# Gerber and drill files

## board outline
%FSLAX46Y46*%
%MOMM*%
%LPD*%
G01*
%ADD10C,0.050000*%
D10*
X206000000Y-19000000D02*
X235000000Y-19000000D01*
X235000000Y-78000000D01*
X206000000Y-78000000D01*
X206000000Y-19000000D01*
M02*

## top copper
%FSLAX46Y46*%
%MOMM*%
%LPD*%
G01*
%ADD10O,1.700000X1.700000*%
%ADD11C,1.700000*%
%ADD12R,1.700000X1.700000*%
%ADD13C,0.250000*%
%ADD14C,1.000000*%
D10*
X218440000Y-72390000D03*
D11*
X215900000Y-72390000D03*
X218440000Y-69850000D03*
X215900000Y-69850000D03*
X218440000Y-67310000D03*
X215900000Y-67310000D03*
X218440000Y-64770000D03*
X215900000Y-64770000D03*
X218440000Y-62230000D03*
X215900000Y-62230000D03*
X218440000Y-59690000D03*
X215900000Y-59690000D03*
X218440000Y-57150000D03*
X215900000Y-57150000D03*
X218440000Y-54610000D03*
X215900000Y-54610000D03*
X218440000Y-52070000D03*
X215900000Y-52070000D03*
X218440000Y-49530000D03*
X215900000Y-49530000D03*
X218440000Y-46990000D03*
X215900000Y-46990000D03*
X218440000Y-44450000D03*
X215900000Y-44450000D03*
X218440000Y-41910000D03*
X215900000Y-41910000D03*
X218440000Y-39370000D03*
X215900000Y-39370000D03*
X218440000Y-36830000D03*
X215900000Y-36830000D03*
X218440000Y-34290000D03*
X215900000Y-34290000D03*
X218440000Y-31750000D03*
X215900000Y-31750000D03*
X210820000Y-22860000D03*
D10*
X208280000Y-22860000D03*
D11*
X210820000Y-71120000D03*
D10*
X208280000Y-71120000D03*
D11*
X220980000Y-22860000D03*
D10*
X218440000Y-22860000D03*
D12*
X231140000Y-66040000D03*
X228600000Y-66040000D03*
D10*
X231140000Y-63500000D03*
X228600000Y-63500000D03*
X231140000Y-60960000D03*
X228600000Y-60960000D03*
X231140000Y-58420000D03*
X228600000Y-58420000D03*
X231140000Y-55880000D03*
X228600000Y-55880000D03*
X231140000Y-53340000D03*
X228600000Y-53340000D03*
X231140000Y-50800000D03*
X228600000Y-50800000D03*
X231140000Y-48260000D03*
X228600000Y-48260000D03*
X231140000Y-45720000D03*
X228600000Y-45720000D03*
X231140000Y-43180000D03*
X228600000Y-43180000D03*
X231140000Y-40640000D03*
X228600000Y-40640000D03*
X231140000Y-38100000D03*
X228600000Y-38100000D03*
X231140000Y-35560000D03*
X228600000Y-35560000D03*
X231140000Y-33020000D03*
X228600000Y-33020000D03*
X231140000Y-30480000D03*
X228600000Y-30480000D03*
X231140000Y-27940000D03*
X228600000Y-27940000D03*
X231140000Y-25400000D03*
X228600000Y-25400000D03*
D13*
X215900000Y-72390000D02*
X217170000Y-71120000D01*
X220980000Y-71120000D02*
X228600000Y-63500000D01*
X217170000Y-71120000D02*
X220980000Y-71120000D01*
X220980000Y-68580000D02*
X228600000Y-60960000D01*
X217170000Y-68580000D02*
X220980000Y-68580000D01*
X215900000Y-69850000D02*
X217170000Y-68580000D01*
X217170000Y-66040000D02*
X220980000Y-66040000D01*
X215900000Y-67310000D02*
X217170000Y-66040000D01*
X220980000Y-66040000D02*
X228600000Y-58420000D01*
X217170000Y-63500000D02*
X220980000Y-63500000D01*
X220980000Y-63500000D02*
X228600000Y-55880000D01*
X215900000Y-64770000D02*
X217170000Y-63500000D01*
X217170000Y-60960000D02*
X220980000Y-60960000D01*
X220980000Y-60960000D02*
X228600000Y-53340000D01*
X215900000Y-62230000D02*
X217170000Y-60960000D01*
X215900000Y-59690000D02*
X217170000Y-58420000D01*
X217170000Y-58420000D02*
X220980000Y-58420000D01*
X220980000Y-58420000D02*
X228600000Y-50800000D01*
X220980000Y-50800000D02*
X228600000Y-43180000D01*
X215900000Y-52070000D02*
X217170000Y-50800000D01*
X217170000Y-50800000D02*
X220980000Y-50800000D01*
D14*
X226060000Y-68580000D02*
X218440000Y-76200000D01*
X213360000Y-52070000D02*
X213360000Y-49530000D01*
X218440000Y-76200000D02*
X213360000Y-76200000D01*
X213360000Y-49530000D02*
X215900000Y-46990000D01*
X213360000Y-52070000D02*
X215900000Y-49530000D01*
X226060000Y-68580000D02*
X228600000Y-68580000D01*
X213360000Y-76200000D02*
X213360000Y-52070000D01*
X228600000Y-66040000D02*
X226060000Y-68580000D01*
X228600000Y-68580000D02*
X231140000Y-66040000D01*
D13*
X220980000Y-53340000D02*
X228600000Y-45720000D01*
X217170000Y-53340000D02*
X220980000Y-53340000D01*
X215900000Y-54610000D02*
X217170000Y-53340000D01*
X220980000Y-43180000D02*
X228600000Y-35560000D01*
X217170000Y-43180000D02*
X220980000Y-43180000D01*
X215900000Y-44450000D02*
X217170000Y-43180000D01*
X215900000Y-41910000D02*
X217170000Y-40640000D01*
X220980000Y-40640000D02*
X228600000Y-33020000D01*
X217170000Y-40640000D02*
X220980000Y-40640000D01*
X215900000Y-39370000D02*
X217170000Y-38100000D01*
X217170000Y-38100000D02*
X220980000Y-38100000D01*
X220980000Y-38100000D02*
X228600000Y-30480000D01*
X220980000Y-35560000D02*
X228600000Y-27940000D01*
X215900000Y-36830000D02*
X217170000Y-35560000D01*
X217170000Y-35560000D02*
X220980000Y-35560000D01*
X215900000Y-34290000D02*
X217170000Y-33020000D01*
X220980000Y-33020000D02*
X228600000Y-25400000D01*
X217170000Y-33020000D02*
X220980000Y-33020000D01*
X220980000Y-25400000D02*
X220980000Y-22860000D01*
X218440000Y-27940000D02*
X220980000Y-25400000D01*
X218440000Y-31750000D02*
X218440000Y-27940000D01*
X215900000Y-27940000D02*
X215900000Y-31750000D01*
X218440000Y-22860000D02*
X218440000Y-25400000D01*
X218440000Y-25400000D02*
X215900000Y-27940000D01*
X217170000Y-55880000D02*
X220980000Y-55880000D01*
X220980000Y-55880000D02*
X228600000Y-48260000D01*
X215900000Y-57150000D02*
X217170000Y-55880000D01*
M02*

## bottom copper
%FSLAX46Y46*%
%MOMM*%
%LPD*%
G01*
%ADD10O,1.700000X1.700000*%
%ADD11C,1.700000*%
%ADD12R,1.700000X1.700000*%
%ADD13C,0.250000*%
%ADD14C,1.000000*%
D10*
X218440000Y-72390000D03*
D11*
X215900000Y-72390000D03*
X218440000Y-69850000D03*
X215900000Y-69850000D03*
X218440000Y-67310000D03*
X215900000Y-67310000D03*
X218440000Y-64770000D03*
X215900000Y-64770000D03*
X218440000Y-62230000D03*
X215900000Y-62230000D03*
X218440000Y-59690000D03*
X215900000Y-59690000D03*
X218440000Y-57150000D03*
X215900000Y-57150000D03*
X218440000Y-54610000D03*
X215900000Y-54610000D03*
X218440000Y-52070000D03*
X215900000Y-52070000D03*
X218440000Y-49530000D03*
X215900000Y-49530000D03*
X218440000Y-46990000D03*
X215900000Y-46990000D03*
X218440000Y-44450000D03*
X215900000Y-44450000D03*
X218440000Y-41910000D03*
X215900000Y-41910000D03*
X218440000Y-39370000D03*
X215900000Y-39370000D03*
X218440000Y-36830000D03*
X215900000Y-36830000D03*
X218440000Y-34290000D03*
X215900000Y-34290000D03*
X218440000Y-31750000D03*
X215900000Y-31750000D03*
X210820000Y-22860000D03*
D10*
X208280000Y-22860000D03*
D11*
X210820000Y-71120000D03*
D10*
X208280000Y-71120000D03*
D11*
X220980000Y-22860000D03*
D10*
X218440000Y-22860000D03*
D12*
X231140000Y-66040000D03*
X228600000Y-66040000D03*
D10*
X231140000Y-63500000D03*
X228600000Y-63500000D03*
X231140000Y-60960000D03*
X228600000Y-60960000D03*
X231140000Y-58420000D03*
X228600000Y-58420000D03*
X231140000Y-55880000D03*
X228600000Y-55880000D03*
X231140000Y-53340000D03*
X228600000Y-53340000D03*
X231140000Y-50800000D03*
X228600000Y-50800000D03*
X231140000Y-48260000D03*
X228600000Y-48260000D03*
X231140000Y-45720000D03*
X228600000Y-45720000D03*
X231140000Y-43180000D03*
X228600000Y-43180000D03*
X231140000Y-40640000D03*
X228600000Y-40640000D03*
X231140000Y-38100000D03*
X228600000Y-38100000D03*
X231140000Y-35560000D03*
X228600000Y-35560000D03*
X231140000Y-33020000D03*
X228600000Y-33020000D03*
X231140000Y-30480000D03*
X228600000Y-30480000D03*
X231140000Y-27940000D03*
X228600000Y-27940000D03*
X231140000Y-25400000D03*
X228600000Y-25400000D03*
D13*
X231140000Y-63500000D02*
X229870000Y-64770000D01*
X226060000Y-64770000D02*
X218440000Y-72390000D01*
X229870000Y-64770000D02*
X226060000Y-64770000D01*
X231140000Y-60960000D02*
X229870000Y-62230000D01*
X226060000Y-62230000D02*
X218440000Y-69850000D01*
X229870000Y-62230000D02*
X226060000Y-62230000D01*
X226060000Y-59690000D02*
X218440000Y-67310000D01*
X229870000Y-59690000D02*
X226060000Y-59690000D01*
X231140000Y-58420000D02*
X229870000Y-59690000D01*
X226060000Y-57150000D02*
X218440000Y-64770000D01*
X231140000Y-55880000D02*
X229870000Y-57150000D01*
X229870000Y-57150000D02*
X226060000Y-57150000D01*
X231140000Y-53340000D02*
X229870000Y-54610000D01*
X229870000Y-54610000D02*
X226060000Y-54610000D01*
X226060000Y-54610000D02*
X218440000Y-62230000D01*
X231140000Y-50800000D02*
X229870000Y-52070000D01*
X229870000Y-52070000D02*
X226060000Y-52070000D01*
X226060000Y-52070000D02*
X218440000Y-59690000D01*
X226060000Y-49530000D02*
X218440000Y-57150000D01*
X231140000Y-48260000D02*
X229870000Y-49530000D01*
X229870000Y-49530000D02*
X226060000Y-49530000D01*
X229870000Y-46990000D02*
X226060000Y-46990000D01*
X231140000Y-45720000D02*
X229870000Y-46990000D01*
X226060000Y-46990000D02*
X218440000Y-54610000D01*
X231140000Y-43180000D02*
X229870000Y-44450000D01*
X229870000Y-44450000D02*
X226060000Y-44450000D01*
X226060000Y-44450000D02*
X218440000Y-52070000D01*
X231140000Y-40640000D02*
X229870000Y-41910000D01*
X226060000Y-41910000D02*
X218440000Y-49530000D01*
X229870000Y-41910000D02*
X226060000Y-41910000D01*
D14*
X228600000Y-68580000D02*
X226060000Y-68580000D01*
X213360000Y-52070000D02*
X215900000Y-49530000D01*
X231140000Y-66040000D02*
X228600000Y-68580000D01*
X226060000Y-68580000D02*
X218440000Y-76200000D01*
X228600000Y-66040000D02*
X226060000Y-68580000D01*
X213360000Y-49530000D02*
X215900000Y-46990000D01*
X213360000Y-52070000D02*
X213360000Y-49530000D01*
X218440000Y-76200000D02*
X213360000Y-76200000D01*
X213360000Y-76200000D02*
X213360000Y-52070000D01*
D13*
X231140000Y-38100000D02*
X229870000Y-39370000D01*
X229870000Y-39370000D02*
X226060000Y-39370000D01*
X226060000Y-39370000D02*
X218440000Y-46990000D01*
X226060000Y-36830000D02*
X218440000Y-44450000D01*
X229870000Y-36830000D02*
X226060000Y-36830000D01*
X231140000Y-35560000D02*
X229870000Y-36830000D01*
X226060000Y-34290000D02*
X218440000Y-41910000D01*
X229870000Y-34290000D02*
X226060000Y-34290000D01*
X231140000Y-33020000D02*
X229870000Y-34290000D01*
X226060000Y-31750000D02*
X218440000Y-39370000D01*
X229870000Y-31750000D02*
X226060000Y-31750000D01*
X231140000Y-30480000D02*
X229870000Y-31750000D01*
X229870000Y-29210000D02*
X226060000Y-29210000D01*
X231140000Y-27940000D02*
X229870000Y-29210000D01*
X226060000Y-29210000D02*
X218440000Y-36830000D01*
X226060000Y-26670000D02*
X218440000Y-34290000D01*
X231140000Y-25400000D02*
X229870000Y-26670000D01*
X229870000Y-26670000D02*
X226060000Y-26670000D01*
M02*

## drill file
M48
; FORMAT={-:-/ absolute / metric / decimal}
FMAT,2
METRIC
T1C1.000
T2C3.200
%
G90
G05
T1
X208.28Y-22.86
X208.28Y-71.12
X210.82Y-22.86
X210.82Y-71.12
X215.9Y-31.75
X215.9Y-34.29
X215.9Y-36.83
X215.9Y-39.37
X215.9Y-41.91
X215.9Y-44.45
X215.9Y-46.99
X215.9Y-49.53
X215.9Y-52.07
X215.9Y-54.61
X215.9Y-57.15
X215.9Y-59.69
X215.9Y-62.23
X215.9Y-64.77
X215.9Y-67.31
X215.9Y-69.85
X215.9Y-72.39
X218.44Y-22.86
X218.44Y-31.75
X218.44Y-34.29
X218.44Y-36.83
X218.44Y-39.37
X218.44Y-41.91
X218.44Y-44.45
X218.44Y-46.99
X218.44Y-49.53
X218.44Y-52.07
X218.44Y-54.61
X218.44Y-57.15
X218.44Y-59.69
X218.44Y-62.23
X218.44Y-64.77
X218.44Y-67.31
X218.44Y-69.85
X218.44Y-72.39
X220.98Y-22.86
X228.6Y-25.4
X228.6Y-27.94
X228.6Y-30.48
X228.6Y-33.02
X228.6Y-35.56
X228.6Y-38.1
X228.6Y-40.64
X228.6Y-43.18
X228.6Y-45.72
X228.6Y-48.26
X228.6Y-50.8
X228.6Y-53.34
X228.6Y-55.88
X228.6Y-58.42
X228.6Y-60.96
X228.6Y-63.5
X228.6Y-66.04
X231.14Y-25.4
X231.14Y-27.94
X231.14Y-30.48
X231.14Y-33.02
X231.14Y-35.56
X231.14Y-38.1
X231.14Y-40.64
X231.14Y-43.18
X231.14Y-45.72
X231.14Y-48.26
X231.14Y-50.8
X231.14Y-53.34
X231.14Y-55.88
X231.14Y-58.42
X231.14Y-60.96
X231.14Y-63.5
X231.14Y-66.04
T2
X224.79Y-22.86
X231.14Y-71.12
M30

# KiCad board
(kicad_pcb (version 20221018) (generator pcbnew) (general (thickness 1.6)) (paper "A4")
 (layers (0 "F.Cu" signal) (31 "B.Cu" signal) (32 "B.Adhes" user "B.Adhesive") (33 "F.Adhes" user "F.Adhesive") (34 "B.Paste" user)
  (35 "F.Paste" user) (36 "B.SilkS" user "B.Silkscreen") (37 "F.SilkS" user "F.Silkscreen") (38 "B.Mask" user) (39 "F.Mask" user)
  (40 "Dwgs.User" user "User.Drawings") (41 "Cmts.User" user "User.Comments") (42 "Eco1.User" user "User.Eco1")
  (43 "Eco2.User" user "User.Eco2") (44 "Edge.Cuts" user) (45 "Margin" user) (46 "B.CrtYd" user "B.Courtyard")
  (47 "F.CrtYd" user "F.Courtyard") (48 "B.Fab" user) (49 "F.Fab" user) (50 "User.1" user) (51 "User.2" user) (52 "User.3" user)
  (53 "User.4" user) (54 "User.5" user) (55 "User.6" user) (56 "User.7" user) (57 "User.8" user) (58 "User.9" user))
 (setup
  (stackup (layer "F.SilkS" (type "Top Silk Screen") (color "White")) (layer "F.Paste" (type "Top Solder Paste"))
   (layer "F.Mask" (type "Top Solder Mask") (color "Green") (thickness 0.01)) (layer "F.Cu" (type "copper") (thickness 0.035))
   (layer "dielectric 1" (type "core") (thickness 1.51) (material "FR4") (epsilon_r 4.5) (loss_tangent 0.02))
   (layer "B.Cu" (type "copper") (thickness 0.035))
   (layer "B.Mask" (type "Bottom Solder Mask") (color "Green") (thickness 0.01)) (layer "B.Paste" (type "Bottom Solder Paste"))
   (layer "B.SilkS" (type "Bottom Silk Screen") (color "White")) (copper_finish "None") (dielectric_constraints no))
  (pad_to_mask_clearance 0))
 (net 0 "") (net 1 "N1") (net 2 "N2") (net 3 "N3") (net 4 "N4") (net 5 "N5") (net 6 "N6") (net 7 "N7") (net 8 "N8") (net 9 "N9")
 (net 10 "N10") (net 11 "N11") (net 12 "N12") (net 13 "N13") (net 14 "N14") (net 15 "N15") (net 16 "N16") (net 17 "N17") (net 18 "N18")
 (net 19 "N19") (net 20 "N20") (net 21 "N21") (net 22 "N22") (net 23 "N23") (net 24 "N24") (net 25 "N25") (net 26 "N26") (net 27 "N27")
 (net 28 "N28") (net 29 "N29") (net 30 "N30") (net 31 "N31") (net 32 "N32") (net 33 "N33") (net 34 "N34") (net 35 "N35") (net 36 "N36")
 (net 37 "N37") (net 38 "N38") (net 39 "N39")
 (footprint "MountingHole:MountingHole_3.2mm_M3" (layer "F.Cu") (at 224.79 22.86)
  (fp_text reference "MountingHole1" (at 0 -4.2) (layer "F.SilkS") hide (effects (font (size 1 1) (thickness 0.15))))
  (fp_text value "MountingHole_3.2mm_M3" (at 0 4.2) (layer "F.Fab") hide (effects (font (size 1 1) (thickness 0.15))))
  (pad "" np_thru_hole circle (at 0 0) (size 3.2 3.2) (drill 3.2) (layers "F&B.Cu" "*.Mask")))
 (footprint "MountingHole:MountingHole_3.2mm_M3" (layer "F.Cu") (at 231.14 71.12)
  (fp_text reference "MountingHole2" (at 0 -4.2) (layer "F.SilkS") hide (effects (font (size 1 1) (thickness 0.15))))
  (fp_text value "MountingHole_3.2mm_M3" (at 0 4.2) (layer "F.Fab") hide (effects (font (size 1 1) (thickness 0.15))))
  (pad "" np_thru_hole circle (at 0 0) (size 3.2 3.2) (drill 3.2) (layers "*.Cu" "*.Mask")))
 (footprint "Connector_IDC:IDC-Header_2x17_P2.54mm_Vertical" (layer "F.Cu") (at 218.44 72.39 180)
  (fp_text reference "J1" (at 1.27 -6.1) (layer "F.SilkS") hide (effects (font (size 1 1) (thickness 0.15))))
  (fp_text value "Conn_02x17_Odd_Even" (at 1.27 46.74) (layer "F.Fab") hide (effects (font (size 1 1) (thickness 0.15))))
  (pad "1" thru_hole oval (at 0 0 180) (size 1.7 1.7) (drill 1) (layers "*.Cu" "*.Mask") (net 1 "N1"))
  (pad "2" thru_hole circle (at 2.54 0 180) (size 1.7 1.7) (drill 1) (layers "*.Cu" "*.Mask") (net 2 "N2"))
  (pad "3" thru_hole circle (at 0 2.54 180) (size 1.7 1.7) (drill 1) (layers "*.Cu" "*.Mask") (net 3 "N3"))
  (pad "4" thru_hole circle (at 2.54 2.54 180) (size 1.7 1.7) (drill 1) (layers "*.Cu" "*.Mask") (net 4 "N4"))
  (pad "5" thru_hole circle (at 0 5.08 180) (size 1.7 1.7) (drill 1) (layers "*.Cu" "*.Mask") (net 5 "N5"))
  (pad "6" thru_hole circle (at 2.54 5.08 180) (size 1.7 1.7) (drill 1) (layers "*.Cu" "*.Mask") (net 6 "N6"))
  (pad "7" thru_hole circle (at 0 7.62 180) (size 1.7 1.7) (drill 1) (layers "*.Cu" "*.Mask") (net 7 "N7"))
  (pad "8" thru_hole circle (at 2.54 7.62 180) (size 1.7 1.7) (drill 1) (layers "*.Cu" "*.Mask") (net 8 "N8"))
  (pad "9" thru_hole circle (at 0 10.16 180) (size 1.7 1.7) (drill 1) (layers "*.Cu" "*.Mask") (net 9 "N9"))
  (pad "10" thru_hole circle (at 2.54 10.16 180) (size 1.7 1.7) (drill 1) (layers "*.Cu" "*.Mask") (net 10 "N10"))
  (pad "11" thru_hole circle (at 0 12.7 180) (size 1.7 1.7) (drill 1) (layers "*.Cu" "*.Mask") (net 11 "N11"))
  (pad "12" thru_hole circle (at 2.54 12.7 180) (size 1.7 1.7) (drill 1) (layers "*.Cu" "*.Mask") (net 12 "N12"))
  (pad "13" thru_hole circle (at 0 15.24 180) (size 1.7 1.7) (drill 1) (layers "*.Cu" "*.Mask") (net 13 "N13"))
  (pad "14" thru_hole circle (at 2.54 15.24 180) (size 1.7 1.7) (drill 1) (layers "*.Cu" "*.Mask") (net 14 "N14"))
  (pad "15" thru_hole circle (at 0 17.78 180) (size 1.7 1.7) (drill 1) (layers "*.Cu" "*.Mask") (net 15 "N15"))
  (pad "16" thru_hole circle (at 2.54 17.78 180) (size 1.7 1.7) (drill 1) (layers "*.Cu" "*.Mask") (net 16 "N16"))
  (pad "17" thru_hole circle (at 0 20.32 180) (size 1.7 1.7) (drill 1) (layers "*.Cu" "*.Mask") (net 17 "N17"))
  (pad "18" thru_hole circle (at 2.54 20.32 180) (size 1.7 1.7) (drill 1) (layers "*.Cu" "*.Mask") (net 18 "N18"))
  (pad "19" thru_hole circle (at 0 22.86 180) (size 1.7 1.7) (drill 1) (layers "*.Cu" "*.Mask") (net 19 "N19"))
  (pad "20" thru_hole circle (at 2.54 22.86 180) (size 1.7 1.7) (drill 1) (layers "*.Cu" "*.Mask") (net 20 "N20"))
  (pad "21" thru_hole circle (at 0 25.4 180) (size 1.7 1.7) (drill 1) (layers "*.Cu" "*.Mask") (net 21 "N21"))
  (pad "22" thru_hole circle (at 2.54 25.4 180) (size 1.7 1.7) (drill 1) (layers "*.Cu" "*.Mask") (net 20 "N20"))
  (pad "23" thru_hole circle (at 0 27.94 180) (size 1.7 1.7) (drill 1) (layers "*.Cu" "*.Mask") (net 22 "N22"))
  (pad "24" thru_hole circle (at 2.54 27.94 180) (size 1.7 1.7) (drill 1) (layers "*.Cu" "*.Mask") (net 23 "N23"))
  (pad "25" thru_hole circle (at 0 30.48 180) (size 1.7 1.7) (drill 1) (layers "*.Cu" "*.Mask") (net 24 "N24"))
  (pad "26" thru_hole circle (at 2.54 30.48 180) (size 1.7 1.7) (drill 1) (layers "*.Cu" "*.Mask") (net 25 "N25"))
  (pad "27" thru_hole circle (at 0 33.02 180) (size 1.7 1.7) (drill 1) (layers "*.Cu" "*.Mask") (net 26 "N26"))
  (pad "28" thru_hole circle (at 2.54 33.02 180) (size 1.7 1.7) (drill 1) (layers "*.Cu" "*.Mask") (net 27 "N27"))
  (pad "29" thru_hole circle (at 0 35.56 180) (size 1.7 1.7) (drill 1) (layers "*.Cu" "*.Mask") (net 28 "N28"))
  (pad "30" thru_hole circle (at 2.54 35.56 180) (size 1.7 1.7) (drill 1) (layers "*.Cu" "*.Mask") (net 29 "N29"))
  (pad "31" thru_hole circle (at 0 38.1 180) (size 1.7 1.7) (drill 1) (layers "*.Cu" "*.Mask") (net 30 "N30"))
  (pad "32" thru_hole circle (at 2.54 38.1 180) (size 1.7 1.7) (drill 1) (layers "*.Cu" "*.Mask") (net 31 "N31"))
  (pad "33" thru_hole circle (at 0 40.64 180) (size 1.7 1.7) (drill 1) (layers "*.Cu" "*.Mask") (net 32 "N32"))
  (pad "34" thru_hole circle (at 2.54 40.64 180) (size 1.7 1.7) (drill 1) (layers "*.Cu" "*.Mask") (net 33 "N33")))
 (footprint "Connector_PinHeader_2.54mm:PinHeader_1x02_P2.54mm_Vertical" (layer "B.Cu") (at 210.82 22.86 90)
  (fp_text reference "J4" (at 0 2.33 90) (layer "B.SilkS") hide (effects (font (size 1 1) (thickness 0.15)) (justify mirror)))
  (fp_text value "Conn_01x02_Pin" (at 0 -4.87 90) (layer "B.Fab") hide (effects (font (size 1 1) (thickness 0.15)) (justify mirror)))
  (pad "1" thru_hole circle (at 0 0 90) (size 1.7 1.7) (drill 1) (layers "*.Cu" "*.Mask") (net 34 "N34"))
  (pad "2" thru_hole oval (at 0 -2.54 90) (size 1.7 1.7) (drill 1) (layers "*.Cu" "*.Mask") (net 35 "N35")))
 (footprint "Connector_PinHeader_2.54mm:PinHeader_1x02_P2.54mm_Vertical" (layer "B.Cu") (at 210.82 71.12 90)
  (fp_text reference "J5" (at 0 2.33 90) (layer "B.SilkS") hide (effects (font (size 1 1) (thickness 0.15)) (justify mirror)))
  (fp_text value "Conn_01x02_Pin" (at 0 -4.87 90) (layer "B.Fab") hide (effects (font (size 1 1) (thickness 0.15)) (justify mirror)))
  (pad "1" thru_hole circle (at 0 0 90) (size 1.7 1.7) (drill 1) (layers "*.Cu" "*.Mask") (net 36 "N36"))
  (pad "2" thru_hole oval (at 0 -2.54 90) (size 1.7 1.7) (drill 1) (layers "*.Cu" "*.Mask") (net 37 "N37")))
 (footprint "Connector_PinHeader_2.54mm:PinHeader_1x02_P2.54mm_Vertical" (layer "B.Cu") (at 220.98 22.86 90)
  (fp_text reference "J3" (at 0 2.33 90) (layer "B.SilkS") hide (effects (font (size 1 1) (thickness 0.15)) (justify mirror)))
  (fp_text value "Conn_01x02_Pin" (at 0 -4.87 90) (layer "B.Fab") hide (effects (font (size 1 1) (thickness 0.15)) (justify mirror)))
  (pad "1" thru_hole circle (at 0 0 90) (size 1.7 1.7) (drill 1) (layers "*.Cu" "*.Mask") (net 32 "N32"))
  (pad "2" thru_hole oval (at 0 -2.54 90) (size 1.7 1.7) (drill 1) (layers "*.Cu" "*.Mask") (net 33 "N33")))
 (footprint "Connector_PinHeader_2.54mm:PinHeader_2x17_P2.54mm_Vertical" (layer "B.Cu") (at 228.6 66.04)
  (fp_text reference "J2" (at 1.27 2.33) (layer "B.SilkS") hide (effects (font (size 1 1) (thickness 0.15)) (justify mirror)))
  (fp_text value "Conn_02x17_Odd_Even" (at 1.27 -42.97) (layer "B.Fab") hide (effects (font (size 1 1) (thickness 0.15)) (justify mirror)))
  (pad "1" thru_hole rect (at 2.54 0) (size 1.7 1.7) (drill 1) (layers "*.Cu" "*.Mask") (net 20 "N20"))
  (pad "2" thru_hole rect (at 0 0) (size 1.7 1.7) (drill 1) (layers "*.Cu" "*.Mask") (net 20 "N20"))
  (pad "3" thru_hole oval (at 2.54 -2.54) (size 1.7 1.7) (drill 1) (layers "*.Cu" "*.Mask") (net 1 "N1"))
  (pad "4" thru_hole oval (at 0 -2.54) (size 1.7 1.7) (drill 1) (layers "*.Cu" "*.Mask") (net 2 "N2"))
  (pad "5" thru_hole oval (at 2.54 -5.08) (size 1.7 1.7) (drill 1) (layers "*.Cu" "*.Mask") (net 3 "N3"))
  (pad "6" thru_hole oval (at 0 -5.08) (size 1.7 1.7) (drill 1) (layers "*.Cu" "*.Mask") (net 4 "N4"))
  (pad "7" thru_hole oval (at 2.54 -7.62) (size 1.7 1.7) (drill 1) (layers "*.Cu" "*.Mask") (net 5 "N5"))
  (pad "8" thru_hole oval (at 0 -7.62) (size 1.7 1.7) (drill 1) (layers "*.Cu" "*.Mask") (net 6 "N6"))
  (pad "9" thru_hole oval (at 2.54 -10.16) (size 1.7 1.7) (drill 1) (layers "*.Cu" "*.Mask") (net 7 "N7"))
  (pad "10" thru_hole oval (at 0 -10.16) (size 1.7 1.7) (drill 1) (layers "*.Cu" "*.Mask") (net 8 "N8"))
  (pad "11" thru_hole oval (at 2.54 -12.7) (size 1.7 1.7) (drill 1) (layers "*.Cu" "*.Mask") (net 9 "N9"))
  (pad "12" thru_hole oval (at 0 -12.7) (size 1.7 1.7) (drill 1) (layers "*.Cu" "*.Mask") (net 10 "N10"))
  (pad "13" thru_hole oval (at 2.54 -15.24) (size 1.7 1.7) (drill 1) (layers "*.Cu" "*.Mask") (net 11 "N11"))
  (pad "14" thru_hole oval (at 0 -15.24) (size 1.7 1.7) (drill 1) (layers "*.Cu" "*.Mask") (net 12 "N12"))
  (pad "15" thru_hole oval (at 2.54 -17.78) (size 1.7 1.7) (drill 1) (layers "*.Cu" "*.Mask") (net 13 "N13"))
  (pad "16" thru_hole oval (at 0 -17.78) (size 1.7 1.7) (drill 1) (layers "*.Cu" "*.Mask") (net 14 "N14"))
  (pad "17" thru_hole oval (at 2.54 -20.32) (size 1.7 1.7) (drill 1) (layers "*.Cu" "*.Mask") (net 15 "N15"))
  (pad "18" thru_hole oval (at 0 -20.32) (size 1.7 1.7) (drill 1) (layers "*.Cu" "*.Mask") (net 16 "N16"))
  (pad "19" thru_hole oval (at 2.54 -22.86) (size 1.7 1.7) (drill 1) (layers "*.Cu" "*.Mask") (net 17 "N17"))
  (pad "20" thru_hole oval (at 0 -22.86) (size 1.7 1.7) (drill 1) (layers "*.Cu" "*.Mask") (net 18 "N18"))
  (pad "21" thru_hole oval (at 2.54 -25.4) (size 1.7 1.7) (drill 1) (layers "*.Cu" "*.Mask") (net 19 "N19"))
  (pad "22" thru_hole oval (at 0 -25.4) (size 1.7 1.7) (drill 1) (layers "*.Cu" "*.Mask") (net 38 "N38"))
  (pad "23" thru_hole oval (at 2.54 -27.94) (size 1.7 1.7) (drill 1) (layers "*.Cu" "*.Mask") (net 21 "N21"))
  (pad "24" thru_hole oval (at 0 -27.94) (size 1.7 1.7) (drill 1) (layers "*.Cu" "*.Mask") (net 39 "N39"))
  (pad "25" thru_hole oval (at 2.54 -30.48) (size 1.7 1.7) (drill 1) (layers "*.Cu" "*.Mask") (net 22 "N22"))
  (pad "26" thru_hole oval (at 0 -30.48) (size 1.7 1.7) (drill 1) (layers "*.Cu" "*.Mask") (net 23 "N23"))
  (pad "27" thru_hole oval (at 2.54 -33.02) (size 1.7 1.7) (drill 1) (layers "*.Cu" "*.Mask") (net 24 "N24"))
  (pad "28" thru_hole oval (at 0 -33.02) (size 1.7 1.7) (drill 1) (layers "*.Cu" "*.Mask") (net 25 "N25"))
  (pad "29" thru_hole oval (at 2.54 -35.56) (size 1.7 1.7) (drill 1) (layers "*.Cu" "*.Mask") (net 26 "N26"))
  (pad "30" thru_hole oval (at 0 -35.56) (size 1.7 1.7) (drill 1) (layers "*.Cu" "*.Mask") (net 27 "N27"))
  (pad "31" thru_hole oval (at 2.54 -38.1) (size 1.7 1.7) (drill 1) (layers "*.Cu" "*.Mask") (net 28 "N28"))
  (pad "32" thru_hole oval (at 0 -38.1) (size 1.7 1.7) (drill 1) (layers "*.Cu" "*.Mask") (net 29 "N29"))
  (pad "33" thru_hole oval (at 2.54 -40.64) (size 1.7 1.7) (drill 1) (layers "*.Cu" "*.Mask") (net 30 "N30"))
  (pad "34" thru_hole oval (at 0 -40.64) (size 1.7 1.7) (drill 1) (layers "*.Cu" "*.Mask") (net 31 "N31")))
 (gr_rect (start 206 19) (end 235 78) (stroke (width 0.05) (type default)) (fill none) (layer "Edge.Cuts"))
 (segment (start 231.14 63.5) (end 229.87 64.77) (width 0.25) (layer "B.Cu") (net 1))
 (segment (start 226.06 64.77) (end 218.44 72.39) (width 0.25) (layer "B.Cu") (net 1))
 (segment (start 229.87 64.77) (end 226.06 64.77) (width 0.25) (layer "B.Cu") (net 1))
 (segment (start 215.9 72.39) (end 217.17 71.12) (width 0.25) (layer "F.Cu") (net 2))
 (segment (start 220.98 71.12) (end 228.6 63.5) (width 0.25) (layer "F.Cu") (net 2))
 (segment (start 217.17 71.12) (end 220.98 71.12) (width 0.25) (layer "F.Cu") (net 2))
 (segment (start 231.14 60.96) (end 229.87 62.23) (width 0.25) (layer "B.Cu") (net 3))
 (segment (start 226.06 62.23) (end 218.44 69.85) (width 0.25) (layer "B.Cu") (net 3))
 (segment (start 229.87 62.23) (end 226.06 62.23) (width 0.25) (layer "B.Cu") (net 3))
 (segment (start 220.98 68.58) (end 228.6 60.96) (width 0.25) (layer "F.Cu") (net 4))
 (segment (start 217.17 68.58) (end 220.98 68.58) (width 0.25) (layer "F.Cu") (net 4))
 (segment (start 215.9 69.85) (end 217.17 68.58) (width 0.25) (layer "F.Cu") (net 4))
 (segment (start 226.06 59.69) (end 218.44 67.31) (width 0.25) (layer "B.Cu") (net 5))
 (segment (start 229.87 59.69) (end 226.06 59.69) (width 0.25) (layer "B.Cu") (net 5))
 (segment (start 231.14 58.42) (end 229.87 59.69) (width 0.25) (layer "B.Cu") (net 5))
 (segment (start 217.17 66.04) (end 220.98 66.04) (width 0.25) (layer "F.Cu") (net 6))
 (segment (start 215.9 67.31) (end 217.17 66.04) (width 0.25) (layer "F.Cu") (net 6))
 (segment (start 220.98 66.04) (end 228.6 58.42) (width 0.25) (layer "F.Cu") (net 6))
 (segment (start 226.06 57.15) (end 218.44 64.77) (width 0.25) (layer "B.Cu") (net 7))
 (segment (start 231.14 55.88) (end 229.87 57.15) (width 0.25) (layer "B.Cu") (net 7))
 (segment (start 229.87 57.15) (end 226.06 57.15) (width 0.25) (layer "B.Cu") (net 7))
 (segment (start 217.17 63.5) (end 220.98 63.5) (width 0.25) (layer "F.Cu") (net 8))
 (segment (start 220.98 63.5) (end 228.6 55.88) (width 0.25) (layer "F.Cu") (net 8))
 (segment (start 215.9 64.77) (end 217.17 63.5) (width 0.25) (layer "F.Cu") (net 8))
 (segment (start 231.14 53.34) (end 229.87 54.61) (width 0.25) (layer "B.Cu") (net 9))
 (segment (start 229.87 54.61) (end 226.06 54.61) (width 0.25) (layer "B.Cu") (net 9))
 (segment (start 226.06 54.61) (end 218.44 62.23) (width 0.25) (layer "B.Cu") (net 9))
 (segment (start 217.17 60.96) (end 220.98 60.96) (width 0.25) (layer "F.Cu") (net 10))
 (segment (start 220.98 60.96) (end 228.6 53.34) (width 0.25) (layer "F.Cu") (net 10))
 (segment (start 215.9 62.23) (end 217.17 60.96) (width 0.25) (layer "F.Cu") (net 10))
 (segment (start 231.14 50.8) (end 229.87 52.07) (width 0.25) (layer "B.Cu") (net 11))
 (segment (start 229.87 52.07) (end 226.06 52.07) (width 0.25) (layer "B.Cu") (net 11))
 (segment (start 226.06 52.07) (end 218.44 59.69) (width 0.25) (layer "B.Cu") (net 11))
 (segment (start 215.9 59.69) (end 217.17 58.42) (width 0.25) (layer "F.Cu") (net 12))
 (segment (start 217.17 58.42) (end 220.98 58.42) (width 0.25) (layer "F.Cu") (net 12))
 (segment (start 220.98 58.42) (end 228.6 50.8) (width 0.25) (layer "F.Cu") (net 12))
 (segment (start 226.06 49.53) (end 218.44 57.15) (width 0.25) (layer "B.Cu") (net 13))
 (segment (start 231.14 48.26) (end 229.87 49.53) (width 0.25) (layer "B.Cu") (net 13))
 (segment (start 229.87 49.53) (end 226.06 49.53) (width 0.25) (layer "B.Cu") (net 13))
 (segment (start 229.87 46.99) (end 226.06 46.99) (width 0.25) (layer "B.Cu") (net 15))
 (segment (start 231.14 45.72) (end 229.87 46.99) (width 0.25) (layer "B.Cu") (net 15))
 (segment (start 226.06 46.99) (end 218.44 54.61) (width 0.25) (layer "B.Cu") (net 15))
 (segment (start 231.14 43.18) (end 229.87 44.45) (width 0.25) (layer "B.Cu") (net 17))
 (segment (start 229.87 44.45) (end 226.06 44.45) (width 0.25) (layer "B.Cu") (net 17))
 (segment (start 226.06 44.45) (end 218.44 52.07) (width 0.25) (layer "B.Cu") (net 17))
 (segment (start 220.98 50.8) (end 228.6 43.18) (width 0.25) (layer "F.Cu") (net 18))
 (segment (start 215.9 52.07) (end 217.17 50.8) (width 0.25) (layer "F.Cu") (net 18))
 (segment (start 217.17 50.8) (end 220.98 50.8) (width 0.25) (layer "F.Cu") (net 18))
 (segment (start 231.14 40.64) (end 229.87 41.91) (width 0.25) (layer "B.Cu") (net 19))
 (segment (start 226.06 41.91) (end 218.44 49.53) (width 0.25) (layer "B.Cu") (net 19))
 (segment (start 229.87 41.91) (end 226.06 41.91) (width 0.25) (layer "B.Cu") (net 19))
 (segment (start 226.06 68.58) (end 218.44 76.2) (width 1) (layer "F.Cu") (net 20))
 (segment (start 213.36 52.07) (end 213.36 49.53) (width 1) (layer "F.Cu") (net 20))
 (segment (start 218.44 76.2) (end 213.36 76.2) (width 1) (layer "F.Cu") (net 20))
 (segment (start 213.36 49.53) (end 215.9 46.99) (width 1) (layer "F.Cu") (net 20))
 (segment (start 213.36 52.07) (end 215.9 49.53) (width 1) (layer "F.Cu") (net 20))
 (segment (start 226.06 68.58) (end 228.6 68.58) (width 1) (layer "F.Cu") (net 20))
 (segment (start 213.36 76.2) (end 213.36 52.07) (width 1) (layer "F.Cu") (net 20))
 (segment (start 228.6 66.04) (end 226.06 68.58) (width 1) (layer "F.Cu") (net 20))
 (segment (start 228.6 68.58) (end 231.14 66.04) (width 1) (layer "F.Cu") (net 20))
 (segment (start 228.6 68.58) (end 226.06 68.58) (width 1) (layer "B.Cu") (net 20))
 (segment (start 213.36 52.07) (end 215.9 49.53) (width 1) (layer "B.Cu") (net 20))
 (segment (start 231.14 66.04) (end 228.6 68.58) (width 1) (layer "B.Cu") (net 20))
 (segment (start 226.06 68.58) (end 218.44 76.2) (width 1) (layer "B.Cu") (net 20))
 (segment (start 228.6 66.04) (end 226.06 68.58) (width 1) (layer "B.Cu") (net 20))
 (segment (start 213.36 49.53) (end 215.9 46.99) (width 1) (layer "B.Cu") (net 20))
 (segment (start 213.36 52.07) (end 213.36 49.53) (width 1) (layer "B.Cu") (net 20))
 (segment (start 218.44 76.2) (end 213.36 76.2) (width 1) (layer "B.Cu") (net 20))
 (segment (start 213.36 76.2) (end 213.36 52.07) (width 1) (layer "B.Cu") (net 20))
 (segment (start 231.14 38.1) (end 229.87 39.37) (width 0.25) (layer "B.Cu") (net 21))
 (segment (start 229.87 39.37) (end 226.06 39.37) (width 0.25) (layer "B.Cu") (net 21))
 (segment (start 226.06 39.37) (end 218.44 46.99) (width 0.25) (layer "B.Cu") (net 21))
 (segment (start 220.98 53.34) (end 228.6 45.72) (width 0.25) (layer "F.Cu") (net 16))
 (segment (start 217.17 53.34) (end 220.98 53.34) (width 0.25) (layer "F.Cu") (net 16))
 (segment (start 215.9 54.61) (end 217.17 53.34) (width 0.25) (layer "F.Cu") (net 16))
 (segment (start 226.06 36.83) (end 218.44 44.45) (width 0.25) (layer "B.Cu") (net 22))
 (segment (start 229.87 36.83) (end 226.06 36.83) (width 0.25) (layer "B.Cu") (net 22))
 (segment (start 231.14 35.56) (end 229.87 36.83) (width 0.25) (layer "B.Cu") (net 22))
 (segment (start 220.98 43.18) (end 228.6 35.56) (width 0.25) (layer "F.Cu") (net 23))
 (segment (start 217.17 43.18) (end 220.98 43.18) (width 0.25) (layer "F.Cu") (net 23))
 (segment (start 215.9 44.45) (end 217.17 43.18) (width 0.25) (layer "F.Cu") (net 23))
 (segment (start 226.06 34.29) (end 218.44 41.91) (width 0.25) (layer "B.Cu") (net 24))
 (segment (start 229.87 34.29) (end 226.06 34.29) (width 0.25) (layer "B.Cu") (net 24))
 (segment (start 231.14 33.02) (end 229.87 34.29) (width 0.25) (layer "B.Cu") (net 24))
 (segment (start 215.9 41.91) (end 217.17 40.64) (width 0.25) (layer "F.Cu") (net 25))
 (segment (start 220.98 40.64) (end 228.6 33.02) (width 0.25) (layer "F.Cu") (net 25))
 (segment (start 217.17 40.64) (end 220.98 40.64) (width 0.25) (layer "F.Cu") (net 25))
 (segment (start 226.06 31.75) (end 218.44 39.37) (width 0.25) (layer "B.Cu") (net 26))
 (segment (start 229.87 31.75) (end 226.06 31.75) (width 0.25) (layer "B.Cu") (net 26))
 (segment (start 231.14 30.48) (end 229.87 31.75) (width 0.25) (layer "B.Cu") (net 26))
 (segment (start 215.9 39.37) (end 217.17 38.1) (width 0.25) (layer "F.Cu") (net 27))
 (segment (start 217.17 38.1) (end 220.98 38.1) (width 0.25) (layer "F.Cu") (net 27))
 (segment (start 220.98 38.1) (end 228.6 30.48) (width 0.25) (layer "F.Cu") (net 27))
 (segment (start 229.87 29.21) (end 226.06 29.21) (width 0.25) (layer "B.Cu") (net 28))
 (segment (start 231.14 27.94) (end 229.87 29.21) (width 0.25) (layer "B.Cu") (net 28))
 (segment (start 226.06 29.21) (end 218.44 36.83) (width 0.25) (layer "B.Cu") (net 28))
 (segment (start 220.98 35.56) (end 228.6 27.94) (width 0.25) (layer "F.Cu") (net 29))
 (segment (start 215.9 36.83) (end 217.17 35.56) (width 0.25) (layer "F.Cu") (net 29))
 (segment (start 217.17 35.56) (end 220.98 35.56) (width 0.25) (layer "F.Cu") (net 29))
 (segment (start 226.06 26.67) (end 218.44 34.29) (width 0.25) (layer "B.Cu") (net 30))
 (segment (start 231.14 25.4) (end 229.87 26.67) (width 0.25) (layer "B.Cu") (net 30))
 (segment (start 229.87 26.67) (end 226.06 26.67) (width 0.25) (layer "B.Cu") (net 30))
 (segment (start 215.9 34.29) (end 217.17 33.02) (width 0.25) (layer "F.Cu") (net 31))
 (segment (start 220.98 33.02) (end 228.6 25.4) (width 0.25) (layer "F.Cu") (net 31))
 (segment (start 217.17 33.02) (end 220.98 33.02) (width 0.25) (layer "F.Cu") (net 31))
 (segment (start 220.98 25.4) (end 220.98 22.86) (width 0.25) (layer "F.Cu") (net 32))
 (segment (start 218.44 27.94) (end 220.98 25.4) (width 0.25) (layer "F.Cu") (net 32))
 (segment (start 218.44 31.75) (end 218.44 27.94) (width 0.25) (layer "F.Cu") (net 32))
 (segment (start 215.9 27.94) (end 215.9 31.75) (width 0.25) (layer "F.Cu") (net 33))
 (segment (start 218.44 22.86) (end 218.44 25.4) (width 0.25) (layer "F.Cu") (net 33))
 (segment (start 218.44 25.4) (end 215.9 27.94) (width 0.25) (layer "F.Cu") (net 33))
 (segment (start 217.17 55.88) (end 220.98 55.88) (width 0.25) (layer "F.Cu") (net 14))
 (segment (start 220.98 55.88) (end 228.6 48.26) (width 0.25) (layer "F.Cu") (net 14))
 (segment (start 215.9 57.15) (end 217.17 55.88) (width 0.25) (layer "F.Cu") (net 14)))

